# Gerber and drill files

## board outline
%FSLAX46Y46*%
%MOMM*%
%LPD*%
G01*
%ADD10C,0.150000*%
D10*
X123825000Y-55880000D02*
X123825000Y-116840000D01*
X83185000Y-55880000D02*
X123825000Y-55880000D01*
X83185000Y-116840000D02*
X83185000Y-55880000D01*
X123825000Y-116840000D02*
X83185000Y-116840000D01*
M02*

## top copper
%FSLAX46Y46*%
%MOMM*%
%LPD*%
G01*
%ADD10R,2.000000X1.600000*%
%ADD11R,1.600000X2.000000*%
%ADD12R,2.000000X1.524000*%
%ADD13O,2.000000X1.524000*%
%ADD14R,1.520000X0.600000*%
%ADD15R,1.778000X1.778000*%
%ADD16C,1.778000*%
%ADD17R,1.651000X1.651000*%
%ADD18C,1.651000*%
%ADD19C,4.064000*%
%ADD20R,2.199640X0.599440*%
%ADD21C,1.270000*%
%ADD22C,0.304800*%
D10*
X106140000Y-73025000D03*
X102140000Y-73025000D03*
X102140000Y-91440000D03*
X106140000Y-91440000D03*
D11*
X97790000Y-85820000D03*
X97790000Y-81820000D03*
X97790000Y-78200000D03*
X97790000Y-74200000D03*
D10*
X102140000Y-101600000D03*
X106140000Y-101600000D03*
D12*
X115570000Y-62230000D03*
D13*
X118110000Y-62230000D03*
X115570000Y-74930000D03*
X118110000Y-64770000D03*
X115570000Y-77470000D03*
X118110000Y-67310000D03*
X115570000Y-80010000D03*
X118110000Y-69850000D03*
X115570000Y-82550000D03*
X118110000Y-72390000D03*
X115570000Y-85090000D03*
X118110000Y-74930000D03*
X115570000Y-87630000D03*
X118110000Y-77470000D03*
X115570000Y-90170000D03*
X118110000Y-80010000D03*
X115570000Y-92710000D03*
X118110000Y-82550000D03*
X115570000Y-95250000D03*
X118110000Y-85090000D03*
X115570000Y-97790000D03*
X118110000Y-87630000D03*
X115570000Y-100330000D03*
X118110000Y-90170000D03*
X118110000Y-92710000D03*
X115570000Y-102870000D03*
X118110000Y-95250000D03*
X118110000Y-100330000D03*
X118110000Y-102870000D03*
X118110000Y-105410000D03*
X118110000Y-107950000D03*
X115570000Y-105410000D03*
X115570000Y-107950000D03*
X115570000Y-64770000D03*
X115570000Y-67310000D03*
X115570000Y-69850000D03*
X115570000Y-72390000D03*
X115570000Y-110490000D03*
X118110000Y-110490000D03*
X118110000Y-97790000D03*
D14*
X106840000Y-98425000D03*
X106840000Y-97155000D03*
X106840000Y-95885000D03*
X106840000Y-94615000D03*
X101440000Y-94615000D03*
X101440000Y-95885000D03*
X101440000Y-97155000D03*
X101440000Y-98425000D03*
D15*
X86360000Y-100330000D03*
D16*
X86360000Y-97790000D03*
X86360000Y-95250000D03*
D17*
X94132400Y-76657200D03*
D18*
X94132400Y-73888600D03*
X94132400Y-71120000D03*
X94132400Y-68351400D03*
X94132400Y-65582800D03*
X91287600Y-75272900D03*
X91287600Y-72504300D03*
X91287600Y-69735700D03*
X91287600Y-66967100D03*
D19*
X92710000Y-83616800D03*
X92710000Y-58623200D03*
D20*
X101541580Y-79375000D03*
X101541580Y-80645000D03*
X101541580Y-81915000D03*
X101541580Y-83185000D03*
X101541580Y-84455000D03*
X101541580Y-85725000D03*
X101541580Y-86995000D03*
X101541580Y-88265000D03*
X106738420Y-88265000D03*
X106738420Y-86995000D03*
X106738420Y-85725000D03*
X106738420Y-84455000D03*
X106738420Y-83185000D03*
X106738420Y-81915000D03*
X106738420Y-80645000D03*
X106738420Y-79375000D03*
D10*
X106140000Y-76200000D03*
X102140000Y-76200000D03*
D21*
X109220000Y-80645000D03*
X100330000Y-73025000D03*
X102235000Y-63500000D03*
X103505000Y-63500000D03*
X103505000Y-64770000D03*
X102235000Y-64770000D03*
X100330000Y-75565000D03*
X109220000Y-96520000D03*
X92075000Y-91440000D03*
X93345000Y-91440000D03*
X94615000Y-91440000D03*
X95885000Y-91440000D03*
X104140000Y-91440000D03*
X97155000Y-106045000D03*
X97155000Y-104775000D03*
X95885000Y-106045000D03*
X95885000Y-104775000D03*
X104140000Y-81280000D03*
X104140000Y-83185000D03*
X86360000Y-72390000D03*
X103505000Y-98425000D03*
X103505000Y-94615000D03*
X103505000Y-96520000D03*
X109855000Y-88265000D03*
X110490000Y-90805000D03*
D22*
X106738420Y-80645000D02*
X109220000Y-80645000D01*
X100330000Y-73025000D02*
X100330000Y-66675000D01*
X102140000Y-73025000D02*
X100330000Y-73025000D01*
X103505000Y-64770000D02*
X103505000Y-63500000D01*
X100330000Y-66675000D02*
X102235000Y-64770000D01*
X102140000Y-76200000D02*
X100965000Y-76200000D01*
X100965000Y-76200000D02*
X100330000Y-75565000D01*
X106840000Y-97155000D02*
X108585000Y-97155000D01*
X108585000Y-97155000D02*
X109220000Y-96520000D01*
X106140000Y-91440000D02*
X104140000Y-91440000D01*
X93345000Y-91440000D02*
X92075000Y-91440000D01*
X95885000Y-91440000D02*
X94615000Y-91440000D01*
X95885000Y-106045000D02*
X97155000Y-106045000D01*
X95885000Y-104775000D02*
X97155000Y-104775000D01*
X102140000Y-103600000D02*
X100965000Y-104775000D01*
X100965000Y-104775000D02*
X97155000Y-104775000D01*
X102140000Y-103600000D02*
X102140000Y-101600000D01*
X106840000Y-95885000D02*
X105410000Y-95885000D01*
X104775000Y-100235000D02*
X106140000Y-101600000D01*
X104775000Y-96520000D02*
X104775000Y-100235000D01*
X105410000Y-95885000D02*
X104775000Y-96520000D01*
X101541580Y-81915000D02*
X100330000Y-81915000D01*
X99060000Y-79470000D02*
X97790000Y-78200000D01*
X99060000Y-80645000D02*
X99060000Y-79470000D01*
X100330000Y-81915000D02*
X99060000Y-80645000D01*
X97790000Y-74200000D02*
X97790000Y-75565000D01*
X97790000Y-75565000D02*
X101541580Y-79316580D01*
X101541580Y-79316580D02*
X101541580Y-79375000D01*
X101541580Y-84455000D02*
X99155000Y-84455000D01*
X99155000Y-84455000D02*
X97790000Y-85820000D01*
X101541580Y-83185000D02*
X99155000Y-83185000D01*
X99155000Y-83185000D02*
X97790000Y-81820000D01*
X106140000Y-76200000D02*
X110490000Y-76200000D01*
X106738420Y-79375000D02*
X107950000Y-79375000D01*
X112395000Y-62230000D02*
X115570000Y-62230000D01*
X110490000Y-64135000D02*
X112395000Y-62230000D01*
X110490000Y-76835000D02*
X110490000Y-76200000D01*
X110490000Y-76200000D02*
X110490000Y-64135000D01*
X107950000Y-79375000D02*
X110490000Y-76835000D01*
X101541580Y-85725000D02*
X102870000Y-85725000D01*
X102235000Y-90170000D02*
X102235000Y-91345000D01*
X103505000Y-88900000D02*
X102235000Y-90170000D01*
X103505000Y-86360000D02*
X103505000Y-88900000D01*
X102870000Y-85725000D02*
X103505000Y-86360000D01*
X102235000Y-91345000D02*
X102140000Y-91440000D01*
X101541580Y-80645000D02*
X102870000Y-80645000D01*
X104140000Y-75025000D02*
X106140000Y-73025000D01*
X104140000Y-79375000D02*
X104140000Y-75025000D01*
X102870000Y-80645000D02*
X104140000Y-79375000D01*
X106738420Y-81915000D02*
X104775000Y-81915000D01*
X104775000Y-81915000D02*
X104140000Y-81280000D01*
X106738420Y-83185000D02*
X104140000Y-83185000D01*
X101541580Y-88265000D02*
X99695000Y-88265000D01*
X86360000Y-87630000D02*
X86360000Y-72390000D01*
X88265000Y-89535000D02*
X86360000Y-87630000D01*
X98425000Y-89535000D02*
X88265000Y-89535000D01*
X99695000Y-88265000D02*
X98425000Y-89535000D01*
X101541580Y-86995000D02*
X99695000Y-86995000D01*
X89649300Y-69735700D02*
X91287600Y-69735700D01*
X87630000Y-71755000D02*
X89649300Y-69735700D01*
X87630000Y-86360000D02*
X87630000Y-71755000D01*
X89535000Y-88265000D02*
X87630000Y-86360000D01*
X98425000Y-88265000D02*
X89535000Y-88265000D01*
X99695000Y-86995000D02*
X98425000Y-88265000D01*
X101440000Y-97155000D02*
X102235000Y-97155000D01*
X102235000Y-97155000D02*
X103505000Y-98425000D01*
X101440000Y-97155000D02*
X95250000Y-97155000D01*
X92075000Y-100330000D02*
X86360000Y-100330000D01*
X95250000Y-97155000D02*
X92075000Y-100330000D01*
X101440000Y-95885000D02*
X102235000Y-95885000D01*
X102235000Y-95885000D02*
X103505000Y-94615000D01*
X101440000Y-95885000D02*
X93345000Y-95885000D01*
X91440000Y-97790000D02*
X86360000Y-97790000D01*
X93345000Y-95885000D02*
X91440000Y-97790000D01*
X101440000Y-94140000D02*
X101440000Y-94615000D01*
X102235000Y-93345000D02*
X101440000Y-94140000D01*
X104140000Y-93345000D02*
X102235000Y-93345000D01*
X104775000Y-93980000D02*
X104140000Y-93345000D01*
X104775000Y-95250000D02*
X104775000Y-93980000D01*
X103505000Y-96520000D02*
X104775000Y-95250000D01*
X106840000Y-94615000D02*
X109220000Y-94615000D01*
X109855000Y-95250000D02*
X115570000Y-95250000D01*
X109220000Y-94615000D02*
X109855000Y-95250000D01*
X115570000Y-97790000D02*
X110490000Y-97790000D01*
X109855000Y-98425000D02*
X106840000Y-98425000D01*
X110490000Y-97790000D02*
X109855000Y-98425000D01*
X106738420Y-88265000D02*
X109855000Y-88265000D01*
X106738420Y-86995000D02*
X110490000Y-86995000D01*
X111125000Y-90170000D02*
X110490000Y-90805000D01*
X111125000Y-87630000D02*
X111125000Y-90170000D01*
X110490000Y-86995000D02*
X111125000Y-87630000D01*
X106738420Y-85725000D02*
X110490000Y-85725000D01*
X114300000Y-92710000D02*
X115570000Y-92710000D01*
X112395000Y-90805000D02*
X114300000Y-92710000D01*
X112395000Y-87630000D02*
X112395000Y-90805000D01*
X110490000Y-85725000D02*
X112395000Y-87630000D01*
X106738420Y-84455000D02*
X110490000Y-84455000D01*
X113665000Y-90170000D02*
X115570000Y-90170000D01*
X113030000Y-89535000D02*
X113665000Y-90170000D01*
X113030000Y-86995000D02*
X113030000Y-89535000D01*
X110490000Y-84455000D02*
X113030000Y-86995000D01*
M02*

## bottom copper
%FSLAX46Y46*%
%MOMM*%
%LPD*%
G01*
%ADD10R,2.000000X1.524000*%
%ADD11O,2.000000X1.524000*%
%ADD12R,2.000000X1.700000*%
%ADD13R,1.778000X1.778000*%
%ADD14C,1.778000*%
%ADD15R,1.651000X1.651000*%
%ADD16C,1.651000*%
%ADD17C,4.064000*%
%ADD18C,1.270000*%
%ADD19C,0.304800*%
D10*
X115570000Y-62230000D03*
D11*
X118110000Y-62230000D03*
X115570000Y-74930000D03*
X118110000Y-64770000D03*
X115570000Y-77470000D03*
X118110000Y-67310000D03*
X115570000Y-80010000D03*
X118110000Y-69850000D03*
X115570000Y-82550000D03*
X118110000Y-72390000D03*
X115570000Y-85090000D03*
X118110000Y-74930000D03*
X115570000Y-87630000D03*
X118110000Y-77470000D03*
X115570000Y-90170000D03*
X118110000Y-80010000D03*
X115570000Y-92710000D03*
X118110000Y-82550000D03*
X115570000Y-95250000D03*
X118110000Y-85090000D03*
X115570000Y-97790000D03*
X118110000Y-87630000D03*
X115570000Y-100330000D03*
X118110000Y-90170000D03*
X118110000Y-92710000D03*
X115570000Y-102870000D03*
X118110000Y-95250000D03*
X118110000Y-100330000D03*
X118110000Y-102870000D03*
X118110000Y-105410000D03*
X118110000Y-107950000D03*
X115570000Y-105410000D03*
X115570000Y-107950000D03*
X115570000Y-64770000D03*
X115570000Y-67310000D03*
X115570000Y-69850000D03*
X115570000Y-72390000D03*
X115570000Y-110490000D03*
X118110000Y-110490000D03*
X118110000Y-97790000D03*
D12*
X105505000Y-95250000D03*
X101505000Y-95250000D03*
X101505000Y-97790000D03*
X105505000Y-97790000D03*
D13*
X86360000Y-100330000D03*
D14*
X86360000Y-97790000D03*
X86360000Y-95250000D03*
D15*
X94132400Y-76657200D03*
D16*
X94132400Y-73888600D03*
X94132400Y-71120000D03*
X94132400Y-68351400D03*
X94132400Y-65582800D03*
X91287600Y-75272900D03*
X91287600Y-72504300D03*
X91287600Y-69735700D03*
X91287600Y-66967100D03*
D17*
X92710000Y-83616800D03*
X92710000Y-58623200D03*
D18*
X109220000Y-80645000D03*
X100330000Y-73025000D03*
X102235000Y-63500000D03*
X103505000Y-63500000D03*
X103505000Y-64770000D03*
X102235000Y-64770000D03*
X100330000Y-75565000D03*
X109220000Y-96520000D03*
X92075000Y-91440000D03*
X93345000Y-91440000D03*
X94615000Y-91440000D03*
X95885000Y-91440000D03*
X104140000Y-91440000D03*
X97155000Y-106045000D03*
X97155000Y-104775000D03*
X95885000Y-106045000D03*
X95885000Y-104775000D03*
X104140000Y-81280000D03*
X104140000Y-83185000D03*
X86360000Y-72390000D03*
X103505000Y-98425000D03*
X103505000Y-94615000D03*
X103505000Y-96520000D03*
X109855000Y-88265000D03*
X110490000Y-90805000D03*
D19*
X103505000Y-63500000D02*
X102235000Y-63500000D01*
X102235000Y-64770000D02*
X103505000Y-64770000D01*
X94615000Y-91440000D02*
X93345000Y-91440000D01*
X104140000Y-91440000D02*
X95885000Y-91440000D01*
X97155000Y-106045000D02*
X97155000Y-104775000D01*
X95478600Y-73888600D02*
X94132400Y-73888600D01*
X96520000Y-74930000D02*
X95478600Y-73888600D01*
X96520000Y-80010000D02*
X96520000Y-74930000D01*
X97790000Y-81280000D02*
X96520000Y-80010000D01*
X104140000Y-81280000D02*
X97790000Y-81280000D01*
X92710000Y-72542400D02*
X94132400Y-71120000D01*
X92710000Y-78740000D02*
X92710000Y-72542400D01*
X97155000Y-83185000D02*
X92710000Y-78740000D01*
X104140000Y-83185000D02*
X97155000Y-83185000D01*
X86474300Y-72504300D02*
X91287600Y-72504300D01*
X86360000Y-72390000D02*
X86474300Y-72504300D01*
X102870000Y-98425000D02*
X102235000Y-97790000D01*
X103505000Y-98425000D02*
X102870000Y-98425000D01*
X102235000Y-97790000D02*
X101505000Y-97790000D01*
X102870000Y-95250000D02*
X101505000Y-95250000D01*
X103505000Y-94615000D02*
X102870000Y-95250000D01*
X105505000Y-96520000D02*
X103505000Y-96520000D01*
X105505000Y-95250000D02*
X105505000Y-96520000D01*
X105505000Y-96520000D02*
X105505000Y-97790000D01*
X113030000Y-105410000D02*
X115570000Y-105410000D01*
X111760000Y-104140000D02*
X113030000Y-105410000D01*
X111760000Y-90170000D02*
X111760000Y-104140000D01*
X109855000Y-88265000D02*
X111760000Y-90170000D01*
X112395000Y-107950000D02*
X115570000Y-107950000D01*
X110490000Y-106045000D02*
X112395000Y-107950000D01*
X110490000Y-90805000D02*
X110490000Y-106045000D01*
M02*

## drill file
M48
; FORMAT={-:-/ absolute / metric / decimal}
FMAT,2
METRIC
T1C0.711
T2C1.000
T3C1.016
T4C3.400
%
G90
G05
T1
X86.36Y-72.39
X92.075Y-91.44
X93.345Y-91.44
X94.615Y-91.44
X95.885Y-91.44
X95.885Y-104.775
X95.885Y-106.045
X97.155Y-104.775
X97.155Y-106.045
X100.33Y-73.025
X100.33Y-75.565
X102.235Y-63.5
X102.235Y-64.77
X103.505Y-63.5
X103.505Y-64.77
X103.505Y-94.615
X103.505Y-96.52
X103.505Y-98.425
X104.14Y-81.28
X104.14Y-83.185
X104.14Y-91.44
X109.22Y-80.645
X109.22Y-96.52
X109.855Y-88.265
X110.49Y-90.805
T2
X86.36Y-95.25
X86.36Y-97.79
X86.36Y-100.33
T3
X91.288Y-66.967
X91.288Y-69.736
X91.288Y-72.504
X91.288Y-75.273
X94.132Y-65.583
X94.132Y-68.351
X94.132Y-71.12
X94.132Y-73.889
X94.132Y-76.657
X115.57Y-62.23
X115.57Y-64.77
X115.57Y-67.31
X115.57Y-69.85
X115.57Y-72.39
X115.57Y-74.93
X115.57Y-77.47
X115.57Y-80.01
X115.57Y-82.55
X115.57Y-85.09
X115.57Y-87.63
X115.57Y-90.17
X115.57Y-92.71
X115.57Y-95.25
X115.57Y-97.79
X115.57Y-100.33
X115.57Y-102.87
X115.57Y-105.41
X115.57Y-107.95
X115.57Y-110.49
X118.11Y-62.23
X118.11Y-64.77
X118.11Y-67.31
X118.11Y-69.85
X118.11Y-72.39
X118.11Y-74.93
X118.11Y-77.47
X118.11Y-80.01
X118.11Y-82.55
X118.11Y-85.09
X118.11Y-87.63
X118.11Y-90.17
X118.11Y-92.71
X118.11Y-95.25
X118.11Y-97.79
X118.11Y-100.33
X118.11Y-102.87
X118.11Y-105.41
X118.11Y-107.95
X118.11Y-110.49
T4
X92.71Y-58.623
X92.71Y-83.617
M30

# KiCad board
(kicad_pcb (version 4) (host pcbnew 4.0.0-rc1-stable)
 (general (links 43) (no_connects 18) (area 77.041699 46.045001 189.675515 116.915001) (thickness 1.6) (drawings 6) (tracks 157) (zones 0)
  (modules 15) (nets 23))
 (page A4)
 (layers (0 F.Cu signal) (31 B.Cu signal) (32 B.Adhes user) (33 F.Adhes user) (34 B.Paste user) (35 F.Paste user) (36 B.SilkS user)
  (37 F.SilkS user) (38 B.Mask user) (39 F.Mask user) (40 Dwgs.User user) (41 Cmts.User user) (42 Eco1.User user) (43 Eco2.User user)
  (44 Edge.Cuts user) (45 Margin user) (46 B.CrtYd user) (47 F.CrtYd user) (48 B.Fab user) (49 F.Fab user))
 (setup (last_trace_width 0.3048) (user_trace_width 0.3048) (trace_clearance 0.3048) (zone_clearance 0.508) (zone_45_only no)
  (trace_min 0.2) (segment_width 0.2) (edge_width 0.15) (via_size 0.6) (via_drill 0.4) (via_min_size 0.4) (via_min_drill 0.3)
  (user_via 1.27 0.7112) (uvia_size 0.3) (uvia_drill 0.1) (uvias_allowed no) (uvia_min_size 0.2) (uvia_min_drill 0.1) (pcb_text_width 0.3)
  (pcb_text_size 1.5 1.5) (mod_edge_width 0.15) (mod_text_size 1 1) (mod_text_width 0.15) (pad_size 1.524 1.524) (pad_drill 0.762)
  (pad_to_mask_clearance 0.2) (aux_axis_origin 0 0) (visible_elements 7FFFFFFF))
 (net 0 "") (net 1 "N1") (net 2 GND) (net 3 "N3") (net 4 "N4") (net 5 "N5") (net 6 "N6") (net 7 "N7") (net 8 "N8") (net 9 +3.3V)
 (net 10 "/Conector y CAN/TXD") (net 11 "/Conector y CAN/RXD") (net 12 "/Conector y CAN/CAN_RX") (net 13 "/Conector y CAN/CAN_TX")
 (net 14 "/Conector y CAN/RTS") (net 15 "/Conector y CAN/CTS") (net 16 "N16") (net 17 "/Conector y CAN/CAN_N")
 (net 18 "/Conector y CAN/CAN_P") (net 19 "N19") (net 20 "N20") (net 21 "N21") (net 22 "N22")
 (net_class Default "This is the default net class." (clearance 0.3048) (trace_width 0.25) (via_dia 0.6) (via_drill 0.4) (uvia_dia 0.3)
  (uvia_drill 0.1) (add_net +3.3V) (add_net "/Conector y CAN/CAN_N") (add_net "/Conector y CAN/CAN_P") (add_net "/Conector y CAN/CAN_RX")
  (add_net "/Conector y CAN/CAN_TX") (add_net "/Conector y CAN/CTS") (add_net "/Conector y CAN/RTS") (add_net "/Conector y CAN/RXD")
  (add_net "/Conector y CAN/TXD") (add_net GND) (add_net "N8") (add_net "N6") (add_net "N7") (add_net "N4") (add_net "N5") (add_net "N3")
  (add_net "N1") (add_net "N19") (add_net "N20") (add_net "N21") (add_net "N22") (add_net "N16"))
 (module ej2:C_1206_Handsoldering (layer F.Cu) (at 104.14 73.025 180)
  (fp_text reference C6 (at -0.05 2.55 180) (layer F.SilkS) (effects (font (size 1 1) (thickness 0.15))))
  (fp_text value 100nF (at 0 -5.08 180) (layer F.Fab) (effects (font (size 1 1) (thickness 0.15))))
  (pad 1 smd rect (at -2 0 180) (size 2 1.6) (layers F.Cu F.Paste F.Mask) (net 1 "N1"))
  (pad 2 smd rect (at 2 0 180) (size 2 1.6) (layers F.Cu F.Paste F.Mask) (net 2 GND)))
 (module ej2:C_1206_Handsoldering (layer F.Cu) (at 104.14 91.44)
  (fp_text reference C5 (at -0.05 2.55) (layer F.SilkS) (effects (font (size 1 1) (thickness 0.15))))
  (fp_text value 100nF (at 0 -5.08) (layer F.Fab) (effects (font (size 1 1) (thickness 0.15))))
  (pad 1 smd rect (at -2 0) (size 2 1.6) (layers F.Cu F.Paste F.Mask) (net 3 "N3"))
  (pad 2 smd rect (at 2 0) (size 2 1.6) (layers F.Cu F.Paste F.Mask) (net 2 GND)))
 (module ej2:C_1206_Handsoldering (layer F.Cu) (at 97.79 83.82 90)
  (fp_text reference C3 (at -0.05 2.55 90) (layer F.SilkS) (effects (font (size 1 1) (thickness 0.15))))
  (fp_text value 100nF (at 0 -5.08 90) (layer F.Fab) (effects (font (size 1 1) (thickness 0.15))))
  (pad 1 smd rect (at -2 0 90) (size 2 1.6) (layers F.Cu F.Paste F.Mask) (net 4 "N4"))
  (pad 2 smd rect (at 2 0 90) (size 2 1.6) (layers F.Cu F.Paste F.Mask) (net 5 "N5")))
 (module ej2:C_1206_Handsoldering (layer F.Cu) (at 97.79 76.2 90)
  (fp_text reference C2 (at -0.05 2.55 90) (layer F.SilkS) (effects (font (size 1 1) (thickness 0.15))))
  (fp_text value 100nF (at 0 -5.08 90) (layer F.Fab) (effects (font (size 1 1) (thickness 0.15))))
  (pad 1 smd rect (at -2 0 90) (size 2 1.6) (layers F.Cu F.Paste F.Mask) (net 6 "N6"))
  (pad 2 smd rect (at 2 0 90) (size 2 1.6) (layers F.Cu F.Paste F.Mask) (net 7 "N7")))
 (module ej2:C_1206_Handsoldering (layer F.Cu) (at 104.14 101.6)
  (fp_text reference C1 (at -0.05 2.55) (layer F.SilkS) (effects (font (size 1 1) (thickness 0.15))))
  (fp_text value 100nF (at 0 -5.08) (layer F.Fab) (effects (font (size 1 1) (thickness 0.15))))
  (pad 1 smd rect (at -2 0) (size 2 1.6) (layers F.Cu F.Paste F.Mask) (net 2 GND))
  (pad 2 smd rect (at 2 0) (size 2 1.6) (layers F.Cu F.Paste F.Mask) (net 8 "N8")))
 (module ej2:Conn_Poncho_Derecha (layer F.Cu) (at 115.57 62.23)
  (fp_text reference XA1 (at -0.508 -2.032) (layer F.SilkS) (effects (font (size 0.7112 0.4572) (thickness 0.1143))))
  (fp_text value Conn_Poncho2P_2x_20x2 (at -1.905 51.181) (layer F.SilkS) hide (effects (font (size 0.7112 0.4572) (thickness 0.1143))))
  (pad 1 thru_hole rect (at 0 0 270) (size 1.524 2) (drill 1.016) (layers *.Cu *.Mask) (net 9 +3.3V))
  (pad 2 thru_hole oval (at 2.54 0 270) (size 1.524 2) (drill 1.016) (layers *.Cu *.Mask))
  (pad 11 thru_hole oval (at 0 12.7 270) (size 1.524 2) (drill 1.016) (layers *.Cu *.Mask))
  (pad 4 thru_hole oval (at 2.54 2.54 270) (size 1.524 2) (drill 1.016) (layers *.Cu *.Mask) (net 2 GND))
  (pad 13 thru_hole oval (at 0 15.24 270) (size 1.524 2) (drill 1.016) (layers *.Cu *.Mask))
  (pad 6 thru_hole oval (at 2.54 5.08 270) (size 1.524 2) (drill 1.016) (layers *.Cu *.Mask))
  (pad 15 thru_hole oval (at 0 17.78 270) (size 1.524 2) (drill 1.016) (layers *.Cu *.Mask))
  (pad 8 thru_hole oval (at 2.54 7.62 270) (size 1.524 2) (drill 1.016) (layers *.Cu *.Mask))
  (pad 17 thru_hole oval (at 0 20.32 270) (size 1.524 2) (drill 1.016) (layers *.Cu *.Mask))
  (pad 10 thru_hole oval (at 2.54 10.16 270) (size 1.524 2) (drill 1.016) (layers *.Cu *.Mask))
  (pad 19 thru_hole oval (at 0 22.86 270) (size 1.524 2) (drill 1.016) (layers *.Cu *.Mask))
  (pad 12 thru_hole oval (at 2.54 12.7 270) (size 1.524 2) (drill 1.016) (layers *.Cu *.Mask))
  (pad 21 thru_hole oval (at 0 25.4 270) (size 1.524 2) (drill 1.016) (layers *.Cu *.Mask))
  (pad 14 thru_hole oval (at 2.54 15.24 270) (size 1.524 2) (drill 1.016) (layers *.Cu *.Mask))
  (pad 23 thru_hole oval (at 0 27.94 270) (size 1.524 2) (drill 1.016) (layers *.Cu *.Mask) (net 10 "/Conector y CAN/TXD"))
  (pad 16 thru_hole oval (at 2.54 17.78 270) (size 1.524 2) (drill 1.016) (layers *.Cu *.Mask))
  (pad 25 thru_hole oval (at 0 30.48 270) (size 1.524 2) (drill 1.016) (layers *.Cu *.Mask) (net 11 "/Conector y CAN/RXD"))
  (pad 18 thru_hole oval (at 2.54 20.32 270) (size 1.524 2) (drill 1.016) (layers *.Cu *.Mask))
  (pad 27 thru_hole oval (at 0 33.02 270) (size 1.524 2) (drill 1.016) (layers *.Cu *.Mask) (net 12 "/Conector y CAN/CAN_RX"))
  (pad 20 thru_hole oval (at 2.54 22.86 270) (size 1.524 2) (drill 1.016) (layers *.Cu *.Mask) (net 2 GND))
  (pad 29 thru_hole oval (at 0 35.56 270) (size 1.524 2) (drill 1.016) (layers *.Cu *.Mask) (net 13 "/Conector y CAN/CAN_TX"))
  (pad 22 thru_hole oval (at 2.54 25.4 270) (size 1.524 2) (drill 1.016) (layers *.Cu *.Mask) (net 2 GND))
  (pad 31 thru_hole oval (at 0 38.1 270) (size 1.524 2) (drill 1.016) (layers *.Cu *.Mask))
  (pad 24 thru_hole oval (at 2.54 27.94 270) (size 1.524 2) (drill 1.016) (layers *.Cu *.Mask) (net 2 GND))
  (pad 26 thru_hole oval (at 2.54 30.48 270) (size 1.524 2) (drill 1.016) (layers *.Cu *.Mask) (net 2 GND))
  (pad 33 thru_hole oval (at 0 40.64 270) (size 1.524 2) (drill 1.016) (layers *.Cu *.Mask))
  (pad 28 thru_hole oval (at 2.54 33.02 270) (size 1.524 2) (drill 1.016) (layers *.Cu *.Mask) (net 2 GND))
  (pad 32 thru_hole oval (at 2.54 38.1 270) (size 1.524 2) (drill 1.016) (layers *.Cu *.Mask) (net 2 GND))
  (pad 34 thru_hole oval (at 2.54 40.64 270) (size 1.524 2) (drill 1.016) (layers *.Cu *.Mask))
  (pad 36 thru_hole oval (at 2.54 43.18 270) (size 1.524 2) (drill 1.016) (layers *.Cu *.Mask))
  (pad 38 thru_hole oval (at 2.54 45.72 270) (size 1.524 2) (drill 1.016) (layers *.Cu *.Mask) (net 2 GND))
  (pad 35 thru_hole oval (at 0 43.18 270) (size 1.524 2) (drill 1.016) (layers *.Cu *.Mask) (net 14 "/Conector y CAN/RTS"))
  (pad 37 thru_hole oval (at 0 45.72 270) (size 1.524 2) (drill 1.016) (layers *.Cu *.Mask) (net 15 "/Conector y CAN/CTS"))
  (pad 3 thru_hole oval (at 0 2.54 270) (size 1.524 2) (drill 1.016) (layers *.Cu *.Mask))
  (pad 5 thru_hole oval (at 0 5.08 270) (size 1.524 2) (drill 1.016) (layers *.Cu *.Mask))
  (pad 7 thru_hole oval (at 0 7.62 270) (size 1.524 2) (drill 1.016) (layers *.Cu *.Mask))
  (pad 9 thru_hole oval (at 0 10.16 270) (size 1.524 2) (drill 1.016) (layers *.Cu *.Mask))
  (pad 39 thru_hole oval (at 0 48.26 270) (size 1.524 2) (drill 1.016) (layers *.Cu *.Mask))
  (pad 40 thru_hole oval (at 2.54 48.26 270) (size 1.524 2) (drill 1.016) (layers *.Cu *.Mask) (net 2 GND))
  (pad 30 thru_hole oval (at 2.54 35.56 270) (size 1.524 2) (drill 1.016) (layers *.Cu *.Mask) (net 2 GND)))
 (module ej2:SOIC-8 (layer F.Cu) (at 104.14 96.52 180)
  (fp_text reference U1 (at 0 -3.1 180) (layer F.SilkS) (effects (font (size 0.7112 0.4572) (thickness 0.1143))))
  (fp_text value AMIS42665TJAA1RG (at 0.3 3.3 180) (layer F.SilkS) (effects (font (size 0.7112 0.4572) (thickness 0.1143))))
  (pad 1 smd rect (at -2.7 -1.905 90) (size 0.6 1.52) (layers F.Cu F.Paste F.Mask) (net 13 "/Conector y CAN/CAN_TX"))
  (pad 2 smd rect (at -2.7 -0.635 90) (size 0.6 1.52) (layers F.Cu F.Paste F.Mask) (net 2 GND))
  (pad 3 smd rect (at -2.7 0.635 90) (size 0.6 1.52) (layers F.Cu F.Paste F.Mask) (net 8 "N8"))
  (pad 4 smd rect (at -2.7 1.905 90) (size 0.6 1.52) (layers F.Cu F.Paste F.Mask) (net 12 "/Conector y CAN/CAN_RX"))
  (pad 5 smd rect (at 2.7 1.905 90) (size 0.6 1.52) (layers F.Cu F.Paste F.Mask) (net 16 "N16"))
  (pad 6 smd rect (at 2.7 0.635 90) (size 0.6 1.52) (layers F.Cu F.Paste F.Mask) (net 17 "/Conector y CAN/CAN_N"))
  (pad 7 smd rect (at 2.7 -0.635 90) (size 0.6 1.52) (layers F.Cu F.Paste F.Mask) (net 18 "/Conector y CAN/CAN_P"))
  (pad 8 smd rect (at 2.7 -1.905 90) (size 0.6 1.52) (layers F.Cu F.Paste F.Mask) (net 2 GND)))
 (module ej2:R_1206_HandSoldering (layer B.Cu) (at 103.505 95.25 180)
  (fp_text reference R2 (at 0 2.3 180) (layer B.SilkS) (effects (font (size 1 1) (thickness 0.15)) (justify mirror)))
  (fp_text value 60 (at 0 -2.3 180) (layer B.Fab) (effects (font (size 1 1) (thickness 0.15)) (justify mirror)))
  (pad 1 smd rect (at -2 0 180) (size 2 1.7) (layers B.Cu B.Paste B.Mask) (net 16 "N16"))
  (pad 2 smd rect (at 2 0 180) (size 2 1.7) (layers B.Cu B.Paste B.Mask) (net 17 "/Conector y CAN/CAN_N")))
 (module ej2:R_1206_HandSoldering (layer B.Cu) (at 103.505 97.79)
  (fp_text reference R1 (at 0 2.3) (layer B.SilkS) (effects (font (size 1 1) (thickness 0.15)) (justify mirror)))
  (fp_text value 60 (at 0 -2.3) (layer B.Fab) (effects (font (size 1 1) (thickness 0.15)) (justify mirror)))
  (pad 1 smd rect (at -2 0) (size 2 1.7) (layers B.Cu B.Paste B.Mask) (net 18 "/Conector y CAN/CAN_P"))
  (pad 2 smd rect (at 2 0) (size 2 1.7) (layers B.Cu B.Paste B.Mask) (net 16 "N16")))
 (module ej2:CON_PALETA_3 (layer F.Cu) (at 86.36 97.79 90)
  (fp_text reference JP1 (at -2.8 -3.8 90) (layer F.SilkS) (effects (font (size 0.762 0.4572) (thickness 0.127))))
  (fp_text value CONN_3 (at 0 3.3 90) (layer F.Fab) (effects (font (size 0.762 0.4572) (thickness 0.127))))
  (pad 1 thru_hole rect (at -2.54 0 90) (size 1.778 1.778) (drill 1) (layers *.Cu *.Mask) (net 18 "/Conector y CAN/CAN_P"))
  (pad 2 thru_hole circle (at 0 0 90) (size 1.778 1.778) (drill 1) (layers *.Cu *.Mask) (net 17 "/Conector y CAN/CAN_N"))
  (pad 3 thru_hole circle (at 2.54 0 90) (size 1.778 1.778) (drill 1) (layers *.Cu *.Mask) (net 2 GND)))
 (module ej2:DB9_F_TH (layer F.Cu) (at 92.71 71.12 90)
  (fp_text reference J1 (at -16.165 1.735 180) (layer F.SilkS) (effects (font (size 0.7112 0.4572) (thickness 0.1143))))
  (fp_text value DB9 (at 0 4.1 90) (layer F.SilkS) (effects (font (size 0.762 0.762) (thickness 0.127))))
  (pad 1 thru_hole rect (at -5.5372 1.4224 90) (size 1.651 1.651) (drill 1.016) (layers *.Cu *.Mask))
  (pad 2 thru_hole circle (at -2.7686 1.4224 90) (size 1.651 1.651) (drill 1.016) (layers *.Cu *.Mask) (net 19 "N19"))
  (pad 3 thru_hole circle (at 0 1.4224 90) (size 1.651 1.651) (drill 1.016) (layers *.Cu *.Mask) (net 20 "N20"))
  (pad 4 thru_hole circle (at 2.7686 1.4224 90) (size 1.651 1.651) (drill 1.016) (layers *.Cu *.Mask))
  (pad 5 thru_hole circle (at 5.5372 1.4224 90) (size 1.651 1.651) (drill 1.016) (layers *.Cu *.Mask) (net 2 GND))
  (pad 6 thru_hole circle (at -4.1529 -1.4224 90) (size 1.651 1.651) (drill 1.016) (layers *.Cu *.Mask))
  (pad 7 thru_hole circle (at -1.3843 -1.4224 90) (size 1.651 1.651) (drill 1.016) (layers *.Cu *.Mask) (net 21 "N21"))
  (pad 8 thru_hole circle (at 1.3843 -1.4224 90) (size 1.651 1.651) (drill 1.016) (layers *.Cu *.Mask) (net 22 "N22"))
  (pad 9 thru_hole circle (at 4.1529 -1.4224 90) (size 1.651 1.651) (drill 1.016) (layers *.Cu *.Mask))
  (pad 10 thru_hole circle (at -12.4968 0 90) (size 4.064 4.064) (drill 3.4) (layers *.Cu *.Mask))
  (pad 11 thru_hole circle (at 12.4968 0 90) (size 4.064 4.064) (drill 3.4) (layers *.Cu *.Mask)))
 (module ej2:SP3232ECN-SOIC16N (layer F.Cu) (at 104.14 83.82 270)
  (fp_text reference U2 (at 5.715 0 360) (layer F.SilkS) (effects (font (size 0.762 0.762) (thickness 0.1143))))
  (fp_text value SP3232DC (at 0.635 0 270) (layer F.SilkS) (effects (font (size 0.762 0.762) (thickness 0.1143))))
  (pad 1 smd rect (at -4.445 2.59842 270) (size 0.59944 2.19964) (layers F.Cu F.Paste F.Mask) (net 7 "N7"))
  (pad 2 smd rect (at -3.175 2.59842 270) (size 0.59944 2.19964) (layers F.Cu F.Paste F.Mask) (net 1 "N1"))
  (pad 3 smd rect (at -1.905 2.59842 270) (size 0.59944 2.19964) (layers F.Cu F.Paste F.Mask) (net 6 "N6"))
  (pad 4 smd rect (at -0.635 2.59842 270) (size 0.59944 2.19964) (layers F.Cu F.Paste F.Mask) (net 5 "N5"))
  (pad 5 smd rect (at 0.635 2.59842 270) (size 0.59944 2.19964) (layers F.Cu F.Paste F.Mask) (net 4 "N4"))
  (pad 6 smd rect (at 1.905 2.59842 270) (size 0.59944 2.19964) (layers F.Cu F.Paste F.Mask) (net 3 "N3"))
  (pad 7 smd rect (at 3.175 2.59842 270) (size 0.59944 2.19964) (layers F.Cu F.Paste F.Mask) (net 22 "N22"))
  (pad 8 smd rect (at 4.445 2.59842 270) (size 0.59944 2.19964) (layers F.Cu F.Paste F.Mask) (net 21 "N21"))
  (pad 9 smd rect (at 4.445 -2.59842 270) (size 0.59944 2.19964) (layers F.Cu F.Paste F.Mask) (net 14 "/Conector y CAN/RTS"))
  (pad 10 smd rect (at 3.175 -2.59842 270) (size 0.59944 2.19964) (layers F.Cu F.Paste F.Mask) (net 15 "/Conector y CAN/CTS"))
  (pad 11 smd rect (at 1.905 -2.59842 270) (size 0.59944 2.19964) (layers F.Cu F.Paste F.Mask) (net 11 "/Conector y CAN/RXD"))
  (pad 12 smd rect (at 0.635 -2.59842 270) (size 0.59944 2.19964) (layers F.Cu F.Paste F.Mask) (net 10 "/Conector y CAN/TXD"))
  (pad 13 smd rect (at -0.635 -2.59842 270) (size 0.59944 2.19964) (layers F.Cu F.Paste F.Mask) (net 20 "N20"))
  (pad 14 smd rect (at -1.905 -2.59842 270) (size 0.59944 2.19964) (layers F.Cu F.Paste F.Mask) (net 19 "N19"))
  (pad 15 smd rect (at -3.175 -2.59842 270) (size 0.59944 2.19964) (layers F.Cu F.Paste F.Mask) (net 2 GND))
  (pad 16 smd rect (at -4.445 -2.59842 270) (size 0.59944 2.19964) (layers F.Cu F.Paste F.Mask) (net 9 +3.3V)))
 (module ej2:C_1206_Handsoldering (layer F.Cu) (at 104.14 76.2 180)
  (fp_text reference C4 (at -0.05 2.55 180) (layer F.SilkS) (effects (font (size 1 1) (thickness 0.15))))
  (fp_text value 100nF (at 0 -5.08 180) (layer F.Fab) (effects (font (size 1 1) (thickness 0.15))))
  (pad 1 smd rect (at -2 0 180) (size 2 1.6) (layers F.Cu F.Paste F.Mask) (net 9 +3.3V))
  (pad 2 smd rect (at 2 0 180) (size 2 1.6) (layers F.Cu F.Paste F.Mask) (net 2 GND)))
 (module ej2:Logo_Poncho (layer F.Cu) (at 103.505 111.125)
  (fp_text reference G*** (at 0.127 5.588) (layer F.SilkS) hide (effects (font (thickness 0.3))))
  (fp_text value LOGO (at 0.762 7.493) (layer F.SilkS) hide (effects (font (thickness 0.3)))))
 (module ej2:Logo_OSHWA (layer F.Cu) (at 102.87 59.69)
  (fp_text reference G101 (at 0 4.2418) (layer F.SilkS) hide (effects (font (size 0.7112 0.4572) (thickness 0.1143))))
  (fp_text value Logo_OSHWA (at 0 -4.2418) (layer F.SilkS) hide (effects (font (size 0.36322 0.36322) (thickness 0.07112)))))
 (gr_line (start 123.825 55.88) (end 123.825 116.84) (angle 90) (layer Edge.Cuts) (width 0.15))
 (gr_line (start 83.185 55.88) (end 123.825 55.88) (angle 90) (layer Edge.Cuts) (width 0.15))
 (gr_line (start 83.185 116.84) (end 83.185 55.88) (angle 90) (layer Edge.Cuts) (width 0.15))
 (gr_line (start 123.825 116.84) (end 83.185 116.84) (angle 90) (layer Edge.Cuts) (width 0.15))
 (segment (start 106.73842 80.645) (end 109.22 80.645) (width 0.3048) (layer F.Cu) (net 2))
 (via (at 109.22 80.645) (size 1.27) (drill 0.7112) (layers F.Cu B.Cu) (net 2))
 (segment (start 100.33 73.025) (end 100.33 66.675) (width 0.3048) (layer F.Cu) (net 2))
 (via (at 100.33 73.025) (size 1.27) (drill 0.7112) (layers F.Cu B.Cu) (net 2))
 (segment (start 102.14 73.025) (end 100.33 73.025) (width 0.3048) (layer F.Cu) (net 2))
 (via (at 102.235 63.5) (size 1.27) (drill 0.7112) (layers F.Cu B.Cu) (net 2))
 (segment (start 103.505 63.5) (end 102.235 63.5) (width 0.3048) (layer B.Cu) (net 2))
 (via (at 103.505 63.5) (size 1.27) (drill 0.7112) (layers F.Cu B.Cu) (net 2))
 (segment (start 103.505 64.77) (end 103.505 63.5) (width 0.3048) (layer F.Cu) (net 2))
 (via (at 103.505 64.77) (size 1.27) (drill 0.7112) (layers F.Cu B.Cu) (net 2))
 (segment (start 102.235 64.77) (end 103.505 64.77) (width 0.3048) (layer B.Cu) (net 2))
 (via (at 102.235 64.77) (size 1.27) (drill 0.7112) (layers F.Cu B.Cu) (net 2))
 (segment (start 100.33 66.675) (end 102.235 64.77) (width 0.3048) (layer F.Cu) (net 2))
 (segment (start 102.14 76.2) (end 100.965 76.2) (width 0.3048) (layer F.Cu) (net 2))
 (via (at 100.33 75.565) (size 1.27) (drill 0.7112) (layers F.Cu B.Cu) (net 2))
 (segment (start 100.965 76.2) (end 100.33 75.565) (width 0.3048) (layer F.Cu) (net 2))
 (segment (start 106.84 97.155) (end 108.585 97.155) (width 0.3048) (layer F.Cu) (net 2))
 (via (at 109.22 96.52) (size 1.27) (drill 0.7112) (layers F.Cu B.Cu) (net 2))
 (segment (start 108.585 97.155) (end 109.22 96.52) (width 0.3048) (layer F.Cu) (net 2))
 (segment (start 106.14 91.44) (end 104.14 91.44) (width 0.3048) (layer F.Cu) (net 2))
 (via (at 92.075 91.44) (size 1.27) (drill 0.7112) (layers F.Cu B.Cu) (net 2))
 (segment (start 93.345 91.44) (end 92.075 91.44) (width 0.3048) (layer F.Cu) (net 2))
 (via (at 93.345 91.44) (size 1.27) (drill 0.7112) (layers F.Cu B.Cu) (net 2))
 (segment (start 94.615 91.44) (end 93.345 91.44) (width 0.3048) (layer B.Cu) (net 2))
 (via (at 94.615 91.44) (size 1.27) (drill 0.7112) (layers F.Cu B.Cu) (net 2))
 (segment (start 95.885 91.44) (end 94.615 91.44) (width 0.3048) (layer F.Cu) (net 2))
 (via (at 95.885 91.44) (size 1.27) (drill 0.7112) (layers F.Cu B.Cu) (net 2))
 (segment (start 104.14 91.44) (end 95.885 91.44) (width 0.3048) (layer B.Cu) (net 2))
 (via (at 104.14 91.44) (size 1.27) (drill 0.7112) (layers F.Cu B.Cu) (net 2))
 (segment (start 95.885 106.045) (end 97.155 106.045) (width 0.3048) (layer F.Cu) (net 2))
 (via (at 97.155 106.045) (size 1.27) (drill 0.7112) (layers F.Cu B.Cu) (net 2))
 (via (at 97.155 104.775) (size 1.27) (drill 0.7112) (layers F.Cu B.Cu) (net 2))
 (segment (start 97.155 106.045) (end 97.155 104.775) (width 0.3048) (layer B.Cu) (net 2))
 (via (at 95.885 106.045) (size 1.27) (drill 0.7112) (layers F.Cu B.Cu) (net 2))
 (segment (start 95.885 104.775) (end 97.155 104.775) (width 0.3048) (layer F.Cu) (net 2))
 (segment (start 102.14 103.6) (end 100.965 104.775) (width 0.3048) (layer F.Cu) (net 2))
 (segment (start 100.965 104.775) (end 97.155 104.775) (width 0.3048) (layer F.Cu) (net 2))
 (segment (start 102.14 103.6) (end 102.14 101.6) (width 0.3048) (layer F.Cu) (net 2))
 (via (at 95.885 104.775) (size 1.27) (drill 0.7112) (layers F.Cu B.Cu) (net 2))
 (segment (start 106.84 95.885) (end 105.41 95.885) (width 0.3048) (layer F.Cu) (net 8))
 (segment (start 104.775 100.235) (end 106.14 101.6) (width 0.3048) (layer F.Cu) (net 8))
 (segment (start 104.775 96.52) (end 104.775 100.235) (width 0.3048) (layer F.Cu) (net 8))
 (segment (start 105.41 95.885) (end 104.775 96.52) (width 0.3048) (layer F.Cu) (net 8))
 (segment (start 101.54158 81.915) (end 100.33 81.915) (width 0.3048) (layer F.Cu) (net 6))
 (segment (start 99.06 79.47) (end 97.79 78.2) (width 0.3048) (layer F.Cu) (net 6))
 (segment (start 99.06 80.645) (end 99.06 79.47) (width 0.3048) (layer F.Cu) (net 6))
 (segment (start 100.33 81.915) (end 99.06 80.645) (width 0.3048) (layer F.Cu) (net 6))
 (segment (start 97.79 74.2) (end 97.79 75.565) (width 0.3048) (layer F.Cu) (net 7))
 (segment (start 97.79 75.565) (end 101.54158 79.31658) (width 0.3048) (layer F.Cu) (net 7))
 (segment (start 101.54158 79.31658) (end 101.54158 79.375) (width 0.3048) (layer F.Cu) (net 7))
 (segment (start 101.54158 84.455) (end 99.155 84.455) (width 0.3048) (layer F.Cu) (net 4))
 (segment (start 99.155 84.455) (end 97.79 85.82) (width 0.3048) (layer F.Cu) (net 4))
 (segment (start 101.54158 83.185) (end 99.155 83.185) (width 0.3048) (layer F.Cu) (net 5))
 (segment (start 99.155 83.185) (end 97.79 81.82) (width 0.3048) (layer F.Cu) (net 5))
 (segment (start 106.14 76.2) (end 110.49 76.2) (width 0.3048) (layer F.Cu) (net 9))
 (segment (start 106.73842 79.375) (end 107.95 79.375) (width 0.3048) (layer F.Cu) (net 9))
 (segment (start 112.395 62.23) (end 115.57 62.23) (width 0.3048) (layer F.Cu) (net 9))
 (segment (start 110.49 64.135) (end 112.395 62.23) (width 0.3048) (layer F.Cu) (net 9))
 (segment (start 110.49 76.835) (end 110.49 76.2) (width 0.3048) (layer F.Cu) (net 9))
 (segment (start 110.49 76.2) (end 110.49 64.135) (width 0.3048) (layer F.Cu) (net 9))
 (segment (start 107.95 79.375) (end 110.49 76.835) (width 0.3048) (layer F.Cu) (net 9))
 (segment (start 101.54158 85.725) (end 102.87 85.725) (width 0.3048) (layer F.Cu) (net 3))
 (segment (start 102.235 90.17) (end 102.235 91.345) (width 0.3048) (layer F.Cu) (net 3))
 (segment (start 103.505 88.9) (end 102.235 90.17) (width 0.3048) (layer F.Cu) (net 3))
 (segment (start 103.505 86.36) (end 103.505 88.9) (width 0.3048) (layer F.Cu) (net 3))
 (segment (start 102.87 85.725) (end 103.505 86.36) (width 0.3048) (layer F.Cu) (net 3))
 (segment (start 102.235 91.345) (end 102.14 91.44) (width 0.3048) (layer F.Cu) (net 3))
 (segment (start 101.54158 80.645) (end 102.87 80.645) (width 0.3048) (layer F.Cu) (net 1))
 (segment (start 104.14 75.025) (end 106.14 73.025) (width 0.3048) (layer F.Cu) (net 1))
 (segment (start 104.14 79.375) (end 104.14 75.025) (width 0.3048) (layer F.Cu) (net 1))
 (segment (start 102.87 80.645) (end 104.14 79.375) (width 0.3048) (layer F.Cu) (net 1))
 (segment (start 106.73842 81.915) (end 104.775 81.915) (width 0.3048) (layer F.Cu) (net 19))
 (segment (start 95.4786 73.8886) (end 94.1324 73.8886) (width 0.3048) (layer B.Cu) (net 19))
 (segment (start 96.52 74.93) (end 95.4786 73.8886) (width 0.3048) (layer B.Cu) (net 19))
 (segment (start 96.52 80.01) (end 96.52 74.93) (width 0.3048) (layer B.Cu) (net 19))
 (segment (start 97.79 81.28) (end 96.52 80.01) (width 0.3048) (layer B.Cu) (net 19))
 (segment (start 104.14 81.28) (end 97.79 81.28) (width 0.3048) (layer B.Cu) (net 19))
 (via (at 104.14 81.28) (size 1.27) (drill 0.7112) (layers F.Cu B.Cu) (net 19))
 (segment (start 104.775 81.915) (end 104.14 81.28) (width 0.3048) (layer F.Cu) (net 19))
 (segment (start 106.73842 83.185) (end 104.14 83.185) (width 0.3048) (layer F.Cu) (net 20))
 (segment (start 92.71 72.5424) (end 94.1324 71.12) (width 0.3048) (layer B.Cu) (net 20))
 (segment (start 92.71 78.74) (end 92.71 72.5424) (width 0.3048) (layer B.Cu) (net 20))
 (segment (start 97.155 83.185) (end 92.71 78.74) (width 0.3048) (layer B.Cu) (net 20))
 (segment (start 104.14 83.185) (end 97.155 83.185) (width 0.3048) (layer B.Cu) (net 20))
 (via (at 104.14 83.185) (size 1.27) (drill 0.7112) (layers F.Cu B.Cu) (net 20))
 (segment (start 101.54158 88.265) (end 99.695 88.265) (width 0.3048) (layer F.Cu) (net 21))
 (segment (start 86.4743 72.5043) (end 91.2876 72.5043) (width 0.3048) (layer B.Cu) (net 21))
 (segment (start 86.36 72.39) (end 86.4743 72.5043) (width 0.3048) (layer B.Cu) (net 21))
 (via (at 86.36 72.39) (size 1.27) (drill 0.7112) (layers F.Cu B.Cu) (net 21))
 (segment (start 86.36 87.63) (end 86.36 72.39) (width 0.3048) (layer F.Cu) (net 21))
 (segment (start 88.265 89.535) (end 86.36 87.63) (width 0.3048) (layer F.Cu) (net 21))
 (segment (start 98.425 89.535) (end 88.265 89.535) (width 0.3048) (layer F.Cu) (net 21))
 (segment (start 99.695 88.265) (end 98.425 89.535) (width 0.3048) (layer F.Cu) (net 21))
 (segment (start 101.54158 86.995) (end 99.695 86.995) (width 0.3048) (layer F.Cu) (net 22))
 (segment (start 89.6493 69.7357) (end 91.2876 69.7357) (width 0.3048) (layer F.Cu) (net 22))
 (segment (start 87.63 71.755) (end 89.6493 69.7357) (width 0.3048) (layer F.Cu) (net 22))
 (segment (start 87.63 86.36) (end 87.63 71.755) (width 0.3048) (layer F.Cu) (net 22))
 (segment (start 89.535 88.265) (end 87.63 86.36) (width 0.3048) (layer F.Cu) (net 22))
 (segment (start 98.425 88.265) (end 89.535 88.265) (width 0.3048) (layer F.Cu) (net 22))
 (segment (start 99.695 86.995) (end 98.425 88.265) (width 0.3048) (layer F.Cu) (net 22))
 (segment (start 101.44 97.155) (end 102.235 97.155) (width 0.3048) (layer F.Cu) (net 18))
 (segment (start 102.87 98.425) (end 102.235 97.79) (width 0.3048) (layer B.Cu) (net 18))
 (segment (start 103.505 98.425) (end 102.87 98.425) (width 0.3048) (layer B.Cu) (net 18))
 (via (at 103.505 98.425) (size 1.27) (drill 0.7112) (layers F.Cu B.Cu) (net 18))
 (segment (start 102.235 97.155) (end 103.505 98.425) (width 0.3048) (layer F.Cu) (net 18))
 (segment (start 102.235 97.79) (end 101.505 97.79) (width 0.3048) (layer B.Cu) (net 18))
 (segment (start 101.44 97.155) (end 95.25 97.155) (width 0.3048) (layer F.Cu) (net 18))
 (segment (start 92.075 100.33) (end 86.36 100.33) (width 0.3048) (layer F.Cu) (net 18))
 (segment (start 95.25 97.155) (end 92.075 100.33) (width 0.3048) (layer F.Cu) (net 18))
 (segment (start 101.44 95.885) (end 102.235 95.885) (width 0.3048) (layer F.Cu) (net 17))
 (segment (start 102.87 95.25) (end 101.505 95.25) (width 0.3048) (layer B.Cu) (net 17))
 (segment (start 103.505 94.615) (end 102.87 95.25) (width 0.3048) (layer B.Cu) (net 17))
 (via (at 103.505 94.615) (size 1.27) (drill 0.7112) (layers F.Cu B.Cu) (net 17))
 (segment (start 102.235 95.885) (end 103.505 94.615) (width 0.3048) (layer F.Cu) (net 17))
 (segment (start 101.44 95.885) (end 93.345 95.885) (width 0.3048) (layer F.Cu) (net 17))
 (segment (start 91.44 97.79) (end 86.36 97.79) (width 0.3048) (layer F.Cu) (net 17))
 (segment (start 93.345 95.885) (end 91.44 97.79) (width 0.3048) (layer F.Cu) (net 17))
 (segment (start 105.505 96.52) (end 103.505 96.52) (width 0.3048) (layer B.Cu) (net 16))
 (segment (start 101.44 94.14) (end 101.44 94.615) (width 0.3048) (layer F.Cu) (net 16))
 (segment (start 102.235 93.345) (end 101.44 94.14) (width 0.3048) (layer F.Cu) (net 16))
 (segment (start 104.14 93.345) (end 102.235 93.345) (width 0.3048) (layer F.Cu) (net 16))
 (segment (start 104.775 93.98) (end 104.14 93.345) (width 0.3048) (layer F.Cu) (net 16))
 (segment (start 104.775 95.25) (end 104.775 93.98) (width 0.3048) (layer F.Cu) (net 16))
 (segment (start 103.505 96.52) (end 104.775 95.25) (width 0.3048) (layer F.Cu) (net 16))
 (via (at 103.505 96.52) (size 1.27) (drill 0.7112) (layers F.Cu B.Cu) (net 16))
 (segment (start 105.505 95.25) (end 105.505 96.52) (width 0.3048) (layer B.Cu) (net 16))
 (segment (start 105.505 96.52) (end 105.505 97.79) (width 0.3048) (layer B.Cu) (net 16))
 (segment (start 106.84 94.615) (end 109.22 94.615) (width 0.3048) (layer F.Cu) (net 12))
 (segment (start 109.855 95.25) (end 115.57 95.25) (width 0.3048) (layer F.Cu) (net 12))
 (segment (start 109.22 94.615) (end 109.855 95.25) (width 0.3048) (layer F.Cu) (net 12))
 (segment (start 115.57 97.79) (end 110.49 97.79) (width 0.3048) (layer F.Cu) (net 13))
 (segment (start 109.855 98.425) (end 106.84 98.425) (width 0.3048) (layer F.Cu) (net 13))
 (segment (start 110.49 97.79) (end 109.855 98.425) (width 0.3048) (layer F.Cu) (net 13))
 (segment (start 106.73842 88.265) (end 109.855 88.265) (width 0.3048) (layer F.Cu) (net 14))
 (segment (start 113.03 105.41) (end 115.57 105.41) (width 0.3048) (layer B.Cu) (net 14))
 (segment (start 111.76 104.14) (end 113.03 105.41) (width 0.3048) (layer B.Cu) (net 14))
 (segment (start 111.76 90.17) (end 111.76 104.14) (width 0.3048) (layer B.Cu) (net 14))
 (segment (start 109.855 88.265) (end 111.76 90.17) (width 0.3048) (layer B.Cu) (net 14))
 (via (at 109.855 88.265) (size 1.27) (drill 0.7112) (layers F.Cu B.Cu) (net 14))
 (segment (start 106.73842 86.995) (end 110.49 86.995) (width 0.3048) (layer F.Cu) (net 15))
 (segment (start 112.395 107.95) (end 115.57 107.95) (width 0.3048) (layer B.Cu) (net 15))
 (segment (start 110.49 106.045) (end 112.395 107.95) (width 0.3048) (layer B.Cu) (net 15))
 (segment (start 110.49 90.805) (end 110.49 106.045) (width 0.3048) (layer B.Cu) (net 15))
 (via (at 110.49 90.805) (size 1.27) (drill 0.7112) (layers F.Cu B.Cu) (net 15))
 (segment (start 111.125 90.17) (end 110.49 90.805) (width 0.3048) (layer F.Cu) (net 15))
 (segment (start 111.125 87.63) (end 111.125 90.17) (width 0.3048) (layer F.Cu) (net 15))
 (segment (start 110.49 86.995) (end 111.125 87.63) (width 0.3048) (layer F.Cu) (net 15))
 (segment (start 106.73842 85.725) (end 110.49 85.725) (width 0.3048) (layer F.Cu) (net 11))
 (segment (start 114.3 92.71) (end 115.57 92.71) (width 0.3048) (layer F.Cu) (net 11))
 (segment (start 112.395 90.805) (end 114.3 92.71) (width 0.3048) (layer F.Cu) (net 11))
 (segment (start 112.395 87.63) (end 112.395 90.805) (width 0.3048) (layer F.Cu) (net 11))
 (segment (start 110.49 85.725) (end 112.395 87.63) (width 0.3048) (layer F.Cu) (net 11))
 (segment (start 106.73842 84.455) (end 110.49 84.455) (width 0.3048) (layer F.Cu) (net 10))
 (segment (start 113.665 90.17) (end 115.57 90.17) (width 0.3048) (layer F.Cu) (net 10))
 (segment (start 113.03 89.535) (end 113.665 90.17) (width 0.3048) (layer F.Cu) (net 10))
 (segment (start 113.03 86.995) (end 113.03 89.535) (width 0.3048) (layer F.Cu) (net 10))
 (segment (start 110.49 84.455) (end 113.03 86.995) (width 0.3048) (layer F.Cu) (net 10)))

